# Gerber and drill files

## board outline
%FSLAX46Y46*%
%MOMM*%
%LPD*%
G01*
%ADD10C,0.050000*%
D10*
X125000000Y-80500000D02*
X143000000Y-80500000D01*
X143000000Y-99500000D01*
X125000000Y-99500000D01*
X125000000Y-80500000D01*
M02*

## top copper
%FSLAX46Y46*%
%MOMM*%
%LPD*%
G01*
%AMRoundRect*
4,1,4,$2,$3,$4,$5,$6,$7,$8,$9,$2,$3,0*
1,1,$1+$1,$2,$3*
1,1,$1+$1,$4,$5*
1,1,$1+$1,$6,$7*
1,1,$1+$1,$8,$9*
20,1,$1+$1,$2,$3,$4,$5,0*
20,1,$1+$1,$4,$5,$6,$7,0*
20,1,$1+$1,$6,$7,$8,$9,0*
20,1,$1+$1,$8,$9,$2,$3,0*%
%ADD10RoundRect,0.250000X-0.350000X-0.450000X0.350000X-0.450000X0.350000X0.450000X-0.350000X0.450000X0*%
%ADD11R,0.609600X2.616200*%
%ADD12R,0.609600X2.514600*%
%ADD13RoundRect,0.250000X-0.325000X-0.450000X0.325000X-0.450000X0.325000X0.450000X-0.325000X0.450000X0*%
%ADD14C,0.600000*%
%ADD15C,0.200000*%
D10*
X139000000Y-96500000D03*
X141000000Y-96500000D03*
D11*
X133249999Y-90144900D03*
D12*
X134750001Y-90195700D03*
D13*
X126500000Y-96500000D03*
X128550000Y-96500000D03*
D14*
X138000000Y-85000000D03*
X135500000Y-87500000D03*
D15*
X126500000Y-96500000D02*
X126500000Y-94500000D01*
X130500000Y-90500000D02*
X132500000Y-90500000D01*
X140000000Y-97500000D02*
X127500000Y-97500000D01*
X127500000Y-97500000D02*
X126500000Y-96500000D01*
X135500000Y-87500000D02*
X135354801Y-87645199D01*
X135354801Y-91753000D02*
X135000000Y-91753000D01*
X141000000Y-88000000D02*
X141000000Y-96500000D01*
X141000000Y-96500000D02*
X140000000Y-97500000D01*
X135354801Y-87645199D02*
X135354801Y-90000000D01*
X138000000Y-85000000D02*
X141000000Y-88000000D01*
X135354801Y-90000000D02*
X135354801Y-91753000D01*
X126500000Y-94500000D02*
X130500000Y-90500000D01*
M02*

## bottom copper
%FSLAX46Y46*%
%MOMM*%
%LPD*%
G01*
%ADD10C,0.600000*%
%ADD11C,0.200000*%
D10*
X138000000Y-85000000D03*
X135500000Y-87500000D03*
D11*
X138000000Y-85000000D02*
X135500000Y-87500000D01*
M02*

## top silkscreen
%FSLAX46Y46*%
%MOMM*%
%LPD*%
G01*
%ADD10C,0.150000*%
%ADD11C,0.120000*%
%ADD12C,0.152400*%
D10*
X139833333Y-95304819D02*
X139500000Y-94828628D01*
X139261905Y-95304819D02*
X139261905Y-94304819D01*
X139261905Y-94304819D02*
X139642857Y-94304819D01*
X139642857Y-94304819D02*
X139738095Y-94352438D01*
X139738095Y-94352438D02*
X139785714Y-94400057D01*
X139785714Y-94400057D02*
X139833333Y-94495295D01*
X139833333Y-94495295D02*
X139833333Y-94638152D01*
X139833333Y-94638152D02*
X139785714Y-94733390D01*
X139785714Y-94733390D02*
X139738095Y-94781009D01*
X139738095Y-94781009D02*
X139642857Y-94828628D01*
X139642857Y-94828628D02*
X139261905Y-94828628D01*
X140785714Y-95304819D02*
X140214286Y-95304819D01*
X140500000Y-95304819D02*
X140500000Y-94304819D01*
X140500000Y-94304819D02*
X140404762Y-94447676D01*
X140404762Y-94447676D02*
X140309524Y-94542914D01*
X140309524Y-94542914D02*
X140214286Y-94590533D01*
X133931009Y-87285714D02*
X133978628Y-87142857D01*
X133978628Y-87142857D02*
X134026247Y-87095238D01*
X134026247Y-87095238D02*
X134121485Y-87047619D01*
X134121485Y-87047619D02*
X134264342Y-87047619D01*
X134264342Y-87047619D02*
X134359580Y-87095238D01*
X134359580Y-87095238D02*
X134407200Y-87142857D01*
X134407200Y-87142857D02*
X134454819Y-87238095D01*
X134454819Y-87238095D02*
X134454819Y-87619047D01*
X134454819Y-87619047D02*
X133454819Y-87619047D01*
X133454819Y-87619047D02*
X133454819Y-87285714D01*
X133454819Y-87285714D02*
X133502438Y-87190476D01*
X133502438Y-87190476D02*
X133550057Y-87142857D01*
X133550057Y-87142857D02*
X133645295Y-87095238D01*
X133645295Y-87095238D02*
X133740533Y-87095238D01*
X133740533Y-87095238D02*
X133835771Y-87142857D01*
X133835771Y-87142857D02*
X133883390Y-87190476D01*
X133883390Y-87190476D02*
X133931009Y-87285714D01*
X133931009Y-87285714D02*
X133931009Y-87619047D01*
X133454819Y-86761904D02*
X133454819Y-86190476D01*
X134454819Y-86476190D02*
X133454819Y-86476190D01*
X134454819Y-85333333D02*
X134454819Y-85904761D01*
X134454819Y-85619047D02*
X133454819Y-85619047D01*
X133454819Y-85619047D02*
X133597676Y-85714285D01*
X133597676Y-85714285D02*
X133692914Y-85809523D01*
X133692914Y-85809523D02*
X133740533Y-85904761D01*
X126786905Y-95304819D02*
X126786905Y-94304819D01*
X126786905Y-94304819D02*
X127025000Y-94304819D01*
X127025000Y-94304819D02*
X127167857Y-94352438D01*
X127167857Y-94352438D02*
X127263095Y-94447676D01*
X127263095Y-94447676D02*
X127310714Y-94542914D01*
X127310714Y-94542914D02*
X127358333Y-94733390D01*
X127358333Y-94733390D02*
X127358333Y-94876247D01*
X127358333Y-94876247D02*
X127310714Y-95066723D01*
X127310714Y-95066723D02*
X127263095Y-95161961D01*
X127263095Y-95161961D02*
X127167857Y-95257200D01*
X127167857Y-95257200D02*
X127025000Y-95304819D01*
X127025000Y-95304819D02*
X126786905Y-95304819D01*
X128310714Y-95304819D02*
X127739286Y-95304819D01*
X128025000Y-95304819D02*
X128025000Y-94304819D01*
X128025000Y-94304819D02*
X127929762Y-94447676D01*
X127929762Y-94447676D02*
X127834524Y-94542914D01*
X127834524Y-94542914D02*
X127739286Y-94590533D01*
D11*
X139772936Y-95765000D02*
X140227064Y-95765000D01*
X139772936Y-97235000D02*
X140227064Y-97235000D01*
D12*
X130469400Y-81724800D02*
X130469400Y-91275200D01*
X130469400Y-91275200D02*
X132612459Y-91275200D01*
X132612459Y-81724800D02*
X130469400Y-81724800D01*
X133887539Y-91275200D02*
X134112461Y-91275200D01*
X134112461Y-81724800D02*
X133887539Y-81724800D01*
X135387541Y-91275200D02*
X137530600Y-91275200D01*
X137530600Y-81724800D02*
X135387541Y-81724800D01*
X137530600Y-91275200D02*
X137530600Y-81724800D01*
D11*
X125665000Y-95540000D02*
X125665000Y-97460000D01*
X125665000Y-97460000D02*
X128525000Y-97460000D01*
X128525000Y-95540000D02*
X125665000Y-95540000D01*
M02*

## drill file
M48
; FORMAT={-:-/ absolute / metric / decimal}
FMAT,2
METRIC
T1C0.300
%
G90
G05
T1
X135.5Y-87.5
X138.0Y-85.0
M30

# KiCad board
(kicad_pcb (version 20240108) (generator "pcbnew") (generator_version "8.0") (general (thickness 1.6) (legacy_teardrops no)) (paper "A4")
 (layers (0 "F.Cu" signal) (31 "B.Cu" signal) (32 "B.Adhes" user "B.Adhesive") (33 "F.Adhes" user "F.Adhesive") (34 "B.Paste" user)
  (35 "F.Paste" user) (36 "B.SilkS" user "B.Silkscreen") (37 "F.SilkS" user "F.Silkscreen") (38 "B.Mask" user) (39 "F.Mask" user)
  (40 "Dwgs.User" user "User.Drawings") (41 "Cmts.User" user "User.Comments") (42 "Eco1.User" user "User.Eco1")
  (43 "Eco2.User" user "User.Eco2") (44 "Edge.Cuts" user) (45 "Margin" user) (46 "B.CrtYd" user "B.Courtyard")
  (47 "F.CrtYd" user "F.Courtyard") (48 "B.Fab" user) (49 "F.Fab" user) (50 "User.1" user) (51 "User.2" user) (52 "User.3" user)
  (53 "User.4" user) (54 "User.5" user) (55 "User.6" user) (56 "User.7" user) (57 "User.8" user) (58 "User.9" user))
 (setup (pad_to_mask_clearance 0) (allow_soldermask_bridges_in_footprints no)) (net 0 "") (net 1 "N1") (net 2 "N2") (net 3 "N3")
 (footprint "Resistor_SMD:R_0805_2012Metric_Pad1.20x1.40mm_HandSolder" (layer "F.Cu") (at 140 96.5)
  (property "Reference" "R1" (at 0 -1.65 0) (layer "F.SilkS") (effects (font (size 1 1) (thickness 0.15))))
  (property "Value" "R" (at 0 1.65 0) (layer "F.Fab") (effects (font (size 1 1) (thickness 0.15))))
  (fp_line (start -0.227064 -0.735) (end 0.227064 -0.735) (stroke (width 0.12) (type solid)) (layer "F.SilkS"))
  (fp_line (start -0.227064 0.735) (end 0.227064 0.735) (stroke (width 0.12) (type solid)) (layer "F.SilkS"))
  (pad "1" smd roundrect (at -1 0) (size 1.2 1.4) (layers "F.Cu" "F.Paste" "F.Mask") (roundrect_rratio 0.208333) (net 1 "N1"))
  (pad "2" smd roundrect (at 1 0) (size 1.2 1.4) (layers "F.Cu" "F.Paste" "F.Mask") (roundrect_rratio 0.208333) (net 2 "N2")))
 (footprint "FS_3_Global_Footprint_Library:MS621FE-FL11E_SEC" (layer "F.Cu") (at 134 86.5 90)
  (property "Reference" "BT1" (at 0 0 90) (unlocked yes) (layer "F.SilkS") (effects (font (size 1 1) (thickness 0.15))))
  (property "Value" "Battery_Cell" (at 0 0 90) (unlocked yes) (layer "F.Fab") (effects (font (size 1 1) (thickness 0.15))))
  (fp_line (start 4.7752 -3.5306) (end -4.7752 -3.5306) (stroke (width 0.1524) (type solid)) (layer "F.SilkS"))
  (fp_line (start -4.7752 -3.5306) (end -4.7752 -1.387541) (stroke (width 0.1524) (type solid)) (layer "F.SilkS"))
  (fp_line (start 4.7752 -1.387541) (end 4.7752 -3.5306) (stroke (width 0.1524) (type solid)) (layer "F.SilkS"))
  (fp_line (start -4.7752 -0.112461) (end -4.7752 0.112461) (stroke (width 0.1524) (type solid)) (layer "F.SilkS"))
  (fp_line (start 4.7752 0.112461) (end 4.7752 -0.112461) (stroke (width 0.1524) (type solid)) (layer "F.SilkS"))
  (fp_line (start -4.7752 1.387541) (end -4.7752 3.5306) (stroke (width 0.1524) (type solid)) (layer "F.SilkS"))
  (fp_line (start 4.7752 3.5306) (end 4.7752 1.387541) (stroke (width 0.1524) (type solid)) (layer "F.SilkS"))
  (fp_line (start -4.7752 3.5306) (end 4.7752 3.5306) (stroke (width 0.1524) (type solid)) (layer "F.SilkS"))
  (pad "1" smd rect (at -3.6449 -0.750001 90) (size 2.6162 0.6096) (layers "F.Cu" "F.Paste" "F.Mask") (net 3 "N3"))
  (pad "2" smd rect (at -3.6957 0.750001 90) (size 2.5146 0.6096) (layers "F.Cu" "F.Paste" "F.Mask") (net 1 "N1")))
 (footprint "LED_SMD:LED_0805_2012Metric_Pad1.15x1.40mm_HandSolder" (layer "F.Cu") (at 127.525 96.5)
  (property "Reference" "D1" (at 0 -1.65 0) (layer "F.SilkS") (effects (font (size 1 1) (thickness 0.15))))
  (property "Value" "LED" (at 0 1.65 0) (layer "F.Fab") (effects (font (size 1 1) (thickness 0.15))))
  (fp_line (start -1.86 -0.96) (end -1.86 0.96) (stroke (width 0.12) (type solid)) (layer "F.SilkS"))
  (fp_line (start -1.86 0.96) (end 1 0.96) (stroke (width 0.12) (type solid)) (layer "F.SilkS"))
  (fp_line (start 1 -0.96) (end -1.86 -0.96) (stroke (width 0.12) (type solid)) (layer "F.SilkS"))
  (pad "1" smd roundrect (at -1.025 0) (size 1.15 1.4) (layers "F.Cu" "F.Paste" "F.Mask") (roundrect_rratio 0.217391) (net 2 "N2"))
  (pad "2" smd roundrect (at 1.025 0) (size 1.15 1.4) (layers "F.Cu" "F.Paste" "F.Mask") (roundrect_rratio 0.217391) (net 3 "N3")))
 (gr_rect (start 125 80.5) (end 143 99.5) (stroke (width 0.05) (type default)) (fill none) (layer "Edge.Cuts"))
 (segment (start 126.5 96.5) (end 126.5 94.5) (width 0.2) (layer "F.Cu") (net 2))
 (segment (start 130.5 90.5) (end 132.5 90.5) (width 0.2) (layer "F.Cu") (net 2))
 (segment (start 140 97.5) (end 127.5 97.5) (width 0.2) (layer "F.Cu") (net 2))
 (segment (start 127.5 97.5) (end 126.5 96.5) (width 0.2) (layer "F.Cu") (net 2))
 (segment (start 135.5 87.5) (end 135.354801 87.645199) (width 0.2) (layer "F.Cu") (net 2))
 (segment (start 135.354801 91.753) (end 135 91.753) (width 0.2) (layer "F.Cu") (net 2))
 (segment (start 141 88) (end 141 96.5) (width 0.2) (layer "F.Cu") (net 2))
 (segment (start 141 96.5) (end 140 97.5) (width 0.2) (layer "F.Cu") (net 2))
 (segment (start 135.354801 87.645199) (end 135.354801 90) (width 0.2) (layer "F.Cu") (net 2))
 (segment (start 138 85) (end 141 88) (width 0.2) (layer "F.Cu") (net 2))
 (segment (start 135.354801 90) (end 135.354801 91.753) (width 0.2) (layer "F.Cu") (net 2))
 (segment (start 126.5 94.5) (end 130.5 90.5) (width 0.2) (layer "F.Cu") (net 2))
 (via (at 138 85) (size 0.6) (drill 0.3) (layers "F.Cu" "B.Cu") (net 2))
 (via (at 135.5 87.5) (size 0.6) (drill 0.3) (layers "F.Cu" "B.Cu") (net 2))
 (segment (start 138 85) (end 135.5 87.5) (width 0.2) (layer "B.Cu") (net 2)))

